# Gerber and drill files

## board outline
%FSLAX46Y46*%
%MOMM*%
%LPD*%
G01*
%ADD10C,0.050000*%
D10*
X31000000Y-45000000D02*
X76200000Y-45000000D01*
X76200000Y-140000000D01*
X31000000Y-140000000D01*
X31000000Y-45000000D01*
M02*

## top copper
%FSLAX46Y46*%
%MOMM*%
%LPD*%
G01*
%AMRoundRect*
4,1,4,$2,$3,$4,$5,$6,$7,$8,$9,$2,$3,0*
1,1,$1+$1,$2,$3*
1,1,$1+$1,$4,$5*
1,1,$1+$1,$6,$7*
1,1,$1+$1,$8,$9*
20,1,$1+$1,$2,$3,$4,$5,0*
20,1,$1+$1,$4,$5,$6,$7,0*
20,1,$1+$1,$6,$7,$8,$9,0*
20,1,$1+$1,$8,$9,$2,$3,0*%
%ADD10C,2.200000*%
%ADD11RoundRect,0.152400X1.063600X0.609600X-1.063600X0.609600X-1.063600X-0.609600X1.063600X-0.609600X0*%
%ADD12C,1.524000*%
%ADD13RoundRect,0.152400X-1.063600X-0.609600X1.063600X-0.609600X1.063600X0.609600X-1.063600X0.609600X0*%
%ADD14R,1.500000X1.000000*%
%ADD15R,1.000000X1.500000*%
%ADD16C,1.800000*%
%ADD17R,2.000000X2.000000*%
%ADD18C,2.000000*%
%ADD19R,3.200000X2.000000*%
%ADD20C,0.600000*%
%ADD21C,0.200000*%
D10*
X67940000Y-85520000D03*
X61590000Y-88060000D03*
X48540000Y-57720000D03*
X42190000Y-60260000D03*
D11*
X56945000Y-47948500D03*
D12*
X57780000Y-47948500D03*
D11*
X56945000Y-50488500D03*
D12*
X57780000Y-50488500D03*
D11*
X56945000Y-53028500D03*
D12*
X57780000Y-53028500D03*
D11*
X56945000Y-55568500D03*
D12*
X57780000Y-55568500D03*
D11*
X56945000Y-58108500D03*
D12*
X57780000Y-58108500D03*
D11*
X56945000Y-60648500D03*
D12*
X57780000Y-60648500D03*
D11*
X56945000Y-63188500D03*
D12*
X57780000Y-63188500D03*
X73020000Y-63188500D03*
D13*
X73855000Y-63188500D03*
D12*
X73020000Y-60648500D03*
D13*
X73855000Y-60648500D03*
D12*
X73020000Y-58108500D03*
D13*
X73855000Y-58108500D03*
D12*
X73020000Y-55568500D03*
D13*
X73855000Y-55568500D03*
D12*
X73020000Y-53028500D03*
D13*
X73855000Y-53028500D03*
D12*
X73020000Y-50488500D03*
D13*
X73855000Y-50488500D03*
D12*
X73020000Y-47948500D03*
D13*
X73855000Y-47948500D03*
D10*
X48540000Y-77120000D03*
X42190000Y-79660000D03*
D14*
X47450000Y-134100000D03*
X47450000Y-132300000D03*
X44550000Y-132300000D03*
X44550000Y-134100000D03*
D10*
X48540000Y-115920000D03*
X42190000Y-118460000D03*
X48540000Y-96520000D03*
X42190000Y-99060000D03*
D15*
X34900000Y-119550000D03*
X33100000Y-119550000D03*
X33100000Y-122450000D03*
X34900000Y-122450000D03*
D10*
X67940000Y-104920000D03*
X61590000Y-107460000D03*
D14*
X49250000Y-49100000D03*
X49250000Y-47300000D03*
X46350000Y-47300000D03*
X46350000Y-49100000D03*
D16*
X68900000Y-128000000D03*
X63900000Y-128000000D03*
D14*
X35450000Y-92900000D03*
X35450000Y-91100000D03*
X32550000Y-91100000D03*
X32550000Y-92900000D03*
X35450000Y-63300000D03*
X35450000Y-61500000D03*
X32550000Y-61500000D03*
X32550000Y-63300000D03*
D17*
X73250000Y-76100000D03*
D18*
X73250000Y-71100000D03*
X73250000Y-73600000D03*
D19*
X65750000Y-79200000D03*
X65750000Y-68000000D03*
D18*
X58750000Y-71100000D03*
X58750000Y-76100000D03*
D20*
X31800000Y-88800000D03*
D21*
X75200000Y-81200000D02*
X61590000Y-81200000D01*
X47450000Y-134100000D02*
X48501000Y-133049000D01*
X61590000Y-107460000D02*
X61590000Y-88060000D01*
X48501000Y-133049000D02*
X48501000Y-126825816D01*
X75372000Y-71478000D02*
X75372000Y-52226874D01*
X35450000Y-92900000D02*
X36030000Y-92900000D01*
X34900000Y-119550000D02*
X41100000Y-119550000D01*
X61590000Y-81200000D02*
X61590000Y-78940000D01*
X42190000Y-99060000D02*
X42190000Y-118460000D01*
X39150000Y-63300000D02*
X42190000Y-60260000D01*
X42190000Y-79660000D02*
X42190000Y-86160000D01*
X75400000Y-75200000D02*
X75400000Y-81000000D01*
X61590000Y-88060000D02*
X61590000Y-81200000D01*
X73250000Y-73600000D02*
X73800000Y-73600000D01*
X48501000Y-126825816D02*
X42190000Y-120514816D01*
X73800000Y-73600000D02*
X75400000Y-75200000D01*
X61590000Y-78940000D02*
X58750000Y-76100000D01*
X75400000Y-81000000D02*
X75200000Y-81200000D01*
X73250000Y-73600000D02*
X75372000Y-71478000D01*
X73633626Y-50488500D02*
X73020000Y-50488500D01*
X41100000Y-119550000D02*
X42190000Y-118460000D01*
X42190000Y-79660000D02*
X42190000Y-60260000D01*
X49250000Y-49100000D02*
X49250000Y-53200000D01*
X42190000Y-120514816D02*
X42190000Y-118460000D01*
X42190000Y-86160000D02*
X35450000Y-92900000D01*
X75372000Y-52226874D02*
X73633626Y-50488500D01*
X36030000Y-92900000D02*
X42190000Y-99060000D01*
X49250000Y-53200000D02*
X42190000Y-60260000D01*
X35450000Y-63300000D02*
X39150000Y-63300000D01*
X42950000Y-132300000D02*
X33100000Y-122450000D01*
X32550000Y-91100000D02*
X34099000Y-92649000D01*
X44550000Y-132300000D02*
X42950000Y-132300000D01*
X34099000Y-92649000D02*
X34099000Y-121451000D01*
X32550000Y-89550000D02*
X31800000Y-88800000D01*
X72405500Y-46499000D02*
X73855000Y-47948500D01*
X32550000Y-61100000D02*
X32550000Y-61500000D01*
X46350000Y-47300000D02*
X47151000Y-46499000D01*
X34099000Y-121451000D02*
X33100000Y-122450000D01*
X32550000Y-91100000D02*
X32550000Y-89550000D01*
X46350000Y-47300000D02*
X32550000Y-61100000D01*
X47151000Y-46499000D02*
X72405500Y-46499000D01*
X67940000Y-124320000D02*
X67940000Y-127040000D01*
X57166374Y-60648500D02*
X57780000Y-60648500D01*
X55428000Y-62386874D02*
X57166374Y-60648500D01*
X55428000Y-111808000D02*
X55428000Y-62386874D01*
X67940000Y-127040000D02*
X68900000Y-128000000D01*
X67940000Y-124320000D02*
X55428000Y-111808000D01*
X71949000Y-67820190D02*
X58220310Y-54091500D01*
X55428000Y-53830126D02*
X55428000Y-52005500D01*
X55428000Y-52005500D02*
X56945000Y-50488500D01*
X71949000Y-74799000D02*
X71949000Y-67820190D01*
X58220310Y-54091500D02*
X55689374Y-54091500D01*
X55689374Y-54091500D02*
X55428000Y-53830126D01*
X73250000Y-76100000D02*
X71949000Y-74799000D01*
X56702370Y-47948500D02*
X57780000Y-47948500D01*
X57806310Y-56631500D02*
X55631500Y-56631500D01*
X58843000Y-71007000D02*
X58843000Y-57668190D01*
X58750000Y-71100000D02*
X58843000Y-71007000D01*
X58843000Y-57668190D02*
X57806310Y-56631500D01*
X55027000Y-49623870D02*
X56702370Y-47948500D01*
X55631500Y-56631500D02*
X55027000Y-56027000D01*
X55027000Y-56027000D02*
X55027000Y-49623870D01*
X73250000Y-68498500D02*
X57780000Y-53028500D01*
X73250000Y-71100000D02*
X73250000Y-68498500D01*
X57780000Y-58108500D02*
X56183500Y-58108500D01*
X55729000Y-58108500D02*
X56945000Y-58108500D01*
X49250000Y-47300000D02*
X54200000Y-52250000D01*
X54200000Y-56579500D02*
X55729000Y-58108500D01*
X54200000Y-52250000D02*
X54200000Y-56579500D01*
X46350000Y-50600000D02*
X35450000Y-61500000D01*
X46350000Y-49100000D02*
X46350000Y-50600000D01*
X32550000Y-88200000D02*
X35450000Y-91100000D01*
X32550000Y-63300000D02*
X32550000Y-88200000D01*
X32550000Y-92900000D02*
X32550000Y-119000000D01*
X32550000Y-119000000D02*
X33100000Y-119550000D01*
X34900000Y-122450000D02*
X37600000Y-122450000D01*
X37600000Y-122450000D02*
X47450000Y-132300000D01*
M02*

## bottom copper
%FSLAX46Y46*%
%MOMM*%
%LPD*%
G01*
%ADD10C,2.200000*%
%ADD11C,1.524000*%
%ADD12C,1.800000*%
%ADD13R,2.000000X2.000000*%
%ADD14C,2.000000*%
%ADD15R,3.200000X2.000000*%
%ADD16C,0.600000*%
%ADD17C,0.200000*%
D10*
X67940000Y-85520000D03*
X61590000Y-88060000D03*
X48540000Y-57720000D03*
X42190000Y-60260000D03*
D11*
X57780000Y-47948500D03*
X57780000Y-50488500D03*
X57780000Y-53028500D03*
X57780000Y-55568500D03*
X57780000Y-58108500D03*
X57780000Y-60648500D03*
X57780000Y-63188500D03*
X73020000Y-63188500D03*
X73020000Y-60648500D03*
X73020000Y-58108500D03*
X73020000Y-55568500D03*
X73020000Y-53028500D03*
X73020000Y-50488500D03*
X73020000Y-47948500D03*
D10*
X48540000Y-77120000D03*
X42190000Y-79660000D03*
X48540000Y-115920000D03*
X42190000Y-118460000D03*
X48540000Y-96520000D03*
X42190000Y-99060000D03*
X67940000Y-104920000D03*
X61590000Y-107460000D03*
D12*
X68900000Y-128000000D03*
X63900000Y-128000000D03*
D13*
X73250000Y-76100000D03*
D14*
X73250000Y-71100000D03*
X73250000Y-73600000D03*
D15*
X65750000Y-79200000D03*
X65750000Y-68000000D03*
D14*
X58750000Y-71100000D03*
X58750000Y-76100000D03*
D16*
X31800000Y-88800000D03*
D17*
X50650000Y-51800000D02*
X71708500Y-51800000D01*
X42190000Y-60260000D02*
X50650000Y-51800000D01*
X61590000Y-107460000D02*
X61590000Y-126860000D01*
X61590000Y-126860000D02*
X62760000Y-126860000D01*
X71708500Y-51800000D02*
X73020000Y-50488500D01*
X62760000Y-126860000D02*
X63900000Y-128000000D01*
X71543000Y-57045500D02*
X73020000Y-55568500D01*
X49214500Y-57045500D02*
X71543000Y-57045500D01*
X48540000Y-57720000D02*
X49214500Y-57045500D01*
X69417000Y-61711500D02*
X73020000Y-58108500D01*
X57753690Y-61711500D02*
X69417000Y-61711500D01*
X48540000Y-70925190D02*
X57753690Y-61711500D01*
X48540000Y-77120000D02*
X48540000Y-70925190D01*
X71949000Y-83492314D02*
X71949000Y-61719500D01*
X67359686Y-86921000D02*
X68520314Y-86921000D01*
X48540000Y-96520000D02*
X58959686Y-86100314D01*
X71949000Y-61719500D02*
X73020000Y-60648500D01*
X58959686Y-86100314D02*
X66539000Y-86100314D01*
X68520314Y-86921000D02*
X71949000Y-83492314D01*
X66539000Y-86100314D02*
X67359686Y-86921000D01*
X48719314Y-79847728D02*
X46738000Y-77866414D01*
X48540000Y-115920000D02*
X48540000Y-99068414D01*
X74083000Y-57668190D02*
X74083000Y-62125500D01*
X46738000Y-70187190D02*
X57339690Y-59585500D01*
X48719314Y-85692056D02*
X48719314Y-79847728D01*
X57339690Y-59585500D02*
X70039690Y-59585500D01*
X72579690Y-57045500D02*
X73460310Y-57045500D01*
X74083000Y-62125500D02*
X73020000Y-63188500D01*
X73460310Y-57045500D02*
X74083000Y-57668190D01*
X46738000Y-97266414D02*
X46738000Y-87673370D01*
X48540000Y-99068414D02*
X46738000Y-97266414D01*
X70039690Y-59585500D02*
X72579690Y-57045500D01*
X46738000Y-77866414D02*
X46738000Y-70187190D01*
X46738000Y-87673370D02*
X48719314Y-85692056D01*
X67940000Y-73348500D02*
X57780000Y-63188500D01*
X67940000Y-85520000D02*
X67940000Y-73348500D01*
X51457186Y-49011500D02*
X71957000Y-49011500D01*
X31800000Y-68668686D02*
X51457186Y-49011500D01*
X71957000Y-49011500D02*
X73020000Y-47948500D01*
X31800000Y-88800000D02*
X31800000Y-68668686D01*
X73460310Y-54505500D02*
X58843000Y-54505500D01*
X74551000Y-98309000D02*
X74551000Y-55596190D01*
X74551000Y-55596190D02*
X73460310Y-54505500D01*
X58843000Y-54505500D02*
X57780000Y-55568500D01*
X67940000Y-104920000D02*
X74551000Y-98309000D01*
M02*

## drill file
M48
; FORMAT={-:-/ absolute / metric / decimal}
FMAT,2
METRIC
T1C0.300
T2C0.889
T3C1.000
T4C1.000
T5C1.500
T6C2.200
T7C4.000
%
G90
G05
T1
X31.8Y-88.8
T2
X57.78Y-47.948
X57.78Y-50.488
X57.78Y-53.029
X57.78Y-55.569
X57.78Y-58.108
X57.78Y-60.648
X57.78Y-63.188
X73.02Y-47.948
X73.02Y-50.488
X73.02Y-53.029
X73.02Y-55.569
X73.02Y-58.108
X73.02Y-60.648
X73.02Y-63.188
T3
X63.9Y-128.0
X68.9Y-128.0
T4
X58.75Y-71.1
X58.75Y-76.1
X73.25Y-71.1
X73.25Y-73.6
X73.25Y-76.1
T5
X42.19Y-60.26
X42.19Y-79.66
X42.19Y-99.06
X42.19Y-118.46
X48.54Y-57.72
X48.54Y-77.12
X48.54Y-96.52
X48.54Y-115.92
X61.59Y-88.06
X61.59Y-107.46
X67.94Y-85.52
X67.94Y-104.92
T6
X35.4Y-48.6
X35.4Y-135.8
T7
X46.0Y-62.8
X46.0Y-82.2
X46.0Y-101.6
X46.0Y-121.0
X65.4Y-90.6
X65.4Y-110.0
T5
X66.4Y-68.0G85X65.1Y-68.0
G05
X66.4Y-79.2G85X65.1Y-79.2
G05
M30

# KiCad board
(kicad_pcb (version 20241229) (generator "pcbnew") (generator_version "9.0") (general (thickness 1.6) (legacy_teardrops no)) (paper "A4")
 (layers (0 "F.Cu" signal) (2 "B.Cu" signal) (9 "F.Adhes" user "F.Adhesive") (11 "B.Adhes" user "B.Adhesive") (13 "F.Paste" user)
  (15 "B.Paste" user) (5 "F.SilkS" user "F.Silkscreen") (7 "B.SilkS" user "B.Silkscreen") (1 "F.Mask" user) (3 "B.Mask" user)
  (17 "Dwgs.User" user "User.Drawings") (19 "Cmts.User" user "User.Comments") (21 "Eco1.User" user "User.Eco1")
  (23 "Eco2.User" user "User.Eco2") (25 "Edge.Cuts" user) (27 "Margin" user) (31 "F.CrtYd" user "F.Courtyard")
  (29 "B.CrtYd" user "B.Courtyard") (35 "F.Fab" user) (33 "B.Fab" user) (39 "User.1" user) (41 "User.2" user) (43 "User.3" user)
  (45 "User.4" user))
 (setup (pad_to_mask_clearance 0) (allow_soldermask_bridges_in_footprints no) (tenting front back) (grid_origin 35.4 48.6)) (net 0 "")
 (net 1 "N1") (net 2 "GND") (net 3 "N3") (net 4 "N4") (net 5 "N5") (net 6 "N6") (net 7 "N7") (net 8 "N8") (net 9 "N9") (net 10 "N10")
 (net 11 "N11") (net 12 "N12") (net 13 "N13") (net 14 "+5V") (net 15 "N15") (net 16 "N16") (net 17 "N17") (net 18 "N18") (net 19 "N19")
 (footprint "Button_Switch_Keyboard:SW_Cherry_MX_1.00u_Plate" (layer "F.Cu") (at 67.94 85.52)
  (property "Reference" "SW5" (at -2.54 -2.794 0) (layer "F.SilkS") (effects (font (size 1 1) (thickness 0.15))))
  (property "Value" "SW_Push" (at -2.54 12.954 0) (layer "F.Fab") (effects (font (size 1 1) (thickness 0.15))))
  (pad "" np_thru_hole circle (at -2.54 5.08) (size 4 4) (drill 4) (layers "*.Cu" "*.Mask"))
  (pad "1" thru_hole circle (at 0 0) (size 2.2 2.2) (drill 1.5) (layers "*.Cu" "*.Mask") (remove_unused_layers no) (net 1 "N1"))
  (pad "2" thru_hole circle (at -6.35 2.54) (size 2.2 2.2) (drill 1.5) (layers "*.Cu" "*.Mask") (remove_unused_layers no) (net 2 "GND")))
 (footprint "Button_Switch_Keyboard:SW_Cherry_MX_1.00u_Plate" (layer "F.Cu") (at 48.54 57.72)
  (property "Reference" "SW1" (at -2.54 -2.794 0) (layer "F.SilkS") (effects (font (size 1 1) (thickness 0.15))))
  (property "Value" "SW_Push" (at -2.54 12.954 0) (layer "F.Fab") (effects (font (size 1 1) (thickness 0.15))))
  (pad "" np_thru_hole circle (at -2.54 5.08) (size 4 4) (drill 4) (layers "*.Cu" "*.Mask"))
  (pad "1" thru_hole circle (at 0 0) (size 2.2 2.2) (drill 1.5) (layers "*.Cu" "*.Mask") (remove_unused_layers no) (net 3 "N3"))
  (pad "2" thru_hole circle (at -6.35 2.54) (size 2.2 2.2) (drill 1.5) (layers "*.Cu" "*.Mask") (remove_unused_layers no) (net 2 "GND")))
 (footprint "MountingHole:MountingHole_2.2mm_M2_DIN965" (layer "F.Cu") (at 35.4 135.8)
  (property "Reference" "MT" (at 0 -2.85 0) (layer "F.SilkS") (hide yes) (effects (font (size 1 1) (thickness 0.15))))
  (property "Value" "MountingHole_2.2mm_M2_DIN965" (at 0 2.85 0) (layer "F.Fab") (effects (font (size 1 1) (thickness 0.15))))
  (pad "" np_thru_hole circle (at 0 0) (size 2.2 2.2) (drill 2.2) (layers "*.Cu" "*.Mask")))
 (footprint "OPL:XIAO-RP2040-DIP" (layer "F.Cu") (at 65.4 55.5685)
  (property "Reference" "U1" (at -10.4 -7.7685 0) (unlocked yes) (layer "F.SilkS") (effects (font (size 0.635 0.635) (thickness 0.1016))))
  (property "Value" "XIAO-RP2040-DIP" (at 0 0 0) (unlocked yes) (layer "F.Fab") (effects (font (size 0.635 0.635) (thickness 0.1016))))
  (pad "1" smd roundrect (at -8.455 -7.62 180) (size 2.432 1.524) (layers "F.Cu" "F.Mask") (roundrect_rratio 0.1) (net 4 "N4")
   (thermal_bridge_angle 45))
  (pad "1" thru_hole circle (at -7.62 -7.62 180) (size 1.524 1.524) (drill 0.889) (layers "*.Cu" "*.Mask") (remove_unused_layers no)
   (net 4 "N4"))
  (pad "2" smd roundrect (at -8.455 -5.08 180) (size 2.432 1.524) (layers "F.Cu" "F.Mask") (roundrect_rratio 0.1) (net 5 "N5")
   (thermal_bridge_angle 45))
  (pad "2" thru_hole circle (at -7.62 -5.08 180) (size 1.524 1.524) (drill 0.889) (layers "*.Cu" "*.Mask") (remove_unused_layers no)
   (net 5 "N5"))
  (pad "3" smd roundrect (at -8.455 -2.54 180) (size 2.432 1.524) (layers "F.Cu" "F.Mask") (roundrect_rratio 0.1) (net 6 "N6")
   (thermal_bridge_angle 45))
  (pad "3" thru_hole circle (at -7.62 -2.54 180) (size 1.524 1.524) (drill 0.889) (layers "*.Cu" "*.Mask") (remove_unused_layers no)
   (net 6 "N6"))
  (pad "4" smd roundrect (at -8.455 0 180) (size 2.432 1.524) (layers "F.Cu" "F.Mask") (roundrect_rratio 0.1) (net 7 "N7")
   (thermal_bridge_angle 45))
  (pad "4" thru_hole circle (at -7.62 0 180) (size 1.524 1.524) (drill 0.889) (layers "*.Cu" "*.Mask") (remove_unused_layers no)
   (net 7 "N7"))
  (pad "5" smd roundrect (at -8.455 2.54 180) (size 2.432 1.524) (layers "F.Cu" "F.Mask") (roundrect_rratio 0.1) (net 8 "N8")
   (thermal_bridge_angle 45))
  (pad "5" thru_hole circle (at -7.62 2.54 180) (size 1.524 1.524) (drill 0.889) (layers "*.Cu" "*.Mask") (remove_unused_layers no)
   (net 8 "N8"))
  (pad "6" smd roundrect (at -8.455 5.08 180) (size 2.432 1.524) (layers "F.Cu" "F.Mask") (roundrect_rratio 0.1) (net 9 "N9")
   (thermal_bridge_angle 45))
  (pad "6" thru_hole circle (at -7.62 5.08 180) (size 1.524 1.524) (drill 0.889) (layers "*.Cu" "*.Mask") (remove_unused_layers no)
   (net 9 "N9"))
  (pad "7" smd roundrect (at -8.455 7.62 180) (size 2.432 1.524) (layers "F.Cu" "F.Mask") (roundrect_rratio 0.1) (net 1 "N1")
   (thermal_bridge_angle 45))
  (pad "7" thru_hole circle (at -7.62 7.62 180) (size 1.524 1.524) (drill 0.889) (layers "*.Cu" "*.Mask") (remove_unused_layers no)
   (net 1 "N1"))
  (pad "8" thru_hole circle (at 7.62 7.62) (size 1.524 1.524) (drill 0.889) (layers "*.Cu" "*.Mask") (remove_unused_layers no)
   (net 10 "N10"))
  (pad "8" smd roundrect (at 8.455 7.62) (size 2.432 1.524) (layers "F.Cu" "F.Mask") (roundrect_rratio 0.1) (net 10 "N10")
   (thermal_bridge_angle 45))
  (pad "9" thru_hole circle (at 7.62 5.08) (size 1.524 1.524) (drill 0.889) (layers "*.Cu" "*.Mask") (remove_unused_layers no)
   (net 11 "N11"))
  (pad "9" smd roundrect (at 8.455 5.08) (size 2.432 1.524) (layers "F.Cu" "F.Mask") (roundrect_rratio 0.1) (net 11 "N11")
   (thermal_bridge_angle 45))
  (pad "10" thru_hole circle (at 7.62 2.54) (size 1.524 1.524) (drill 0.889) (layers "*.Cu" "*.Mask") (remove_unused_layers no)
   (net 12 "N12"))
  (pad "10" smd roundrect (at 8.455 2.54) (size 2.432 1.524) (layers "F.Cu" "F.Mask") (roundrect_rratio 0.1) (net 12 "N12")
   (thermal_bridge_angle 45))
  (pad "11" thru_hole circle (at 7.62 0) (size 1.524 1.524) (drill 0.889) (layers "*.Cu" "*.Mask") (remove_unused_layers no) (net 3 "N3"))
  (pad "11" smd roundrect (at 8.455 0) (size 2.432 1.524) (layers "F.Cu" "F.Mask") (roundrect_rratio 0.1) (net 3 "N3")
   (thermal_bridge_angle 45))
  (pad "12" thru_hole circle (at 7.62 -2.54) (size 1.524 1.524) (drill 0.889) (layers "*.Cu" "*.Mask") (remove_unused_layers no)
   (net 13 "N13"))
  (pad "12" smd roundrect (at 8.455 -2.54) (size 2.432 1.524) (layers "F.Cu" "F.Mask") (roundrect_rratio 0.1) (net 13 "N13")
   (thermal_bridge_angle 45))
  (pad "13" thru_hole circle (at 7.62 -5.08) (size 1.524 1.524) (drill 0.889) (layers "*.Cu" "*.Mask") (remove_unused_layers no)
   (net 2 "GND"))
  (pad "13" smd roundrect (at 8.455 -5.08) (size 2.432 1.524) (layers "F.Cu" "F.Mask") (roundrect_rratio 0.1) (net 2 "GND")
   (thermal_bridge_angle 45))
  (pad "14" thru_hole circle (at 7.62 -7.62) (size 1.524 1.524) (drill 0.889) (layers "*.Cu" "*.Mask") (remove_unused_layers no)
   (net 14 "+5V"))
  (pad "14" smd roundrect (at 8.455 -7.62) (size 2.432 1.524) (layers "F.Cu" "F.Mask") (roundrect_rratio 0.1) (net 14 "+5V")
   (thermal_bridge_angle 45)))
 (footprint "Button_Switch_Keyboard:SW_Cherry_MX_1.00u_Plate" (layer "F.Cu") (at 48.54 77.12)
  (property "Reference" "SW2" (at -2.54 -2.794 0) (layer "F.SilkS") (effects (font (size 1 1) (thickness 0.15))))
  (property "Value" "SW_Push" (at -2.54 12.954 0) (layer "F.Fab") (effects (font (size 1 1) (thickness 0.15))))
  (pad "" np_thru_hole circle (at -2.54 5.08) (size 4 4) (drill 4) (layers "*.Cu" "*.Mask"))
  (pad "1" thru_hole circle (at 0 0) (size 2.2 2.2) (drill 1.5) (layers "*.Cu" "*.Mask") (remove_unused_layers no) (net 12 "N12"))
  (pad "2" thru_hole circle (at -6.35 2.54) (size 2.2 2.2) (drill 1.5) (layers "*.Cu" "*.Mask") (remove_unused_layers no) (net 2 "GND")))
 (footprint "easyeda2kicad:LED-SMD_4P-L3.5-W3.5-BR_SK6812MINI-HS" (layer "F.Cu") (at 46 133.2)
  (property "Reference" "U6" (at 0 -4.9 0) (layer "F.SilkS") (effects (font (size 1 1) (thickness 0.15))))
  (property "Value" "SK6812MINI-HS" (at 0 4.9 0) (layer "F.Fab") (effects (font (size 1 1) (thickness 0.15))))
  (pad "1" smd rect (at 1.45 0.9 180) (size 1.5 1) (layers "F.Cu" "F.Mask" "F.Paste") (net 2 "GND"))
  (pad "2" smd rect (at 1.45 -0.9 180) (size 1.5 1) (layers "F.Cu" "F.Mask" "F.Paste") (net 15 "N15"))
  (pad "3" smd rect (at -1.45 -0.9 180) (size 1.5 1) (layers "F.Cu" "F.Mask" "F.Paste") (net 14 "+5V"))
  (pad "4" smd rect (at -1.45 0.9 180) (size 1.5 1) (layers "F.Cu" "F.Mask" "F.Paste") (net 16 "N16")))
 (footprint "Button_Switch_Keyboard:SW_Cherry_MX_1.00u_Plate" (layer "F.Cu") (at 48.54 115.92)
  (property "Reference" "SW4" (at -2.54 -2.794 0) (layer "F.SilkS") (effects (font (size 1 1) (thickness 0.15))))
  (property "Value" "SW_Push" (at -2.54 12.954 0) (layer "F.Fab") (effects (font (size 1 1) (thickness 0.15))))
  (pad "" np_thru_hole circle (at -2.54 5.08) (size 4 4) (drill 4) (layers "*.Cu" "*.Mask"))
  (pad "1" thru_hole circle (at 0 0) (size 2.2 2.2) (drill 1.5) (layers "*.Cu" "*.Mask") (remove_unused_layers no) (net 10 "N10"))
  (pad "2" thru_hole circle (at -6.35 2.54) (size 2.2 2.2) (drill 1.5) (layers "*.Cu" "*.Mask") (remove_unused_layers no) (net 2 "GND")))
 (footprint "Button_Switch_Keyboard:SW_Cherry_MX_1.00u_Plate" (layer "F.Cu") (at 48.54 96.52)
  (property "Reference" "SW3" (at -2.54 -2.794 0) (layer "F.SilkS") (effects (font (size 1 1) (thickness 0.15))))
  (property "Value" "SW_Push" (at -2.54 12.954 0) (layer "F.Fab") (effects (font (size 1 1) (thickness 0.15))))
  (pad "" np_thru_hole circle (at -2.54 5.08) (size 4 4) (drill 4) (layers "*.Cu" "*.Mask"))
  (pad "1" thru_hole circle (at 0 0) (size 2.2 2.2) (drill 1.5) (layers "*.Cu" "*.Mask") (remove_unused_layers no) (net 11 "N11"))
  (pad "2" thru_hole circle (at -6.35 2.54) (size 2.2 2.2) (drill 1.5) (layers "*.Cu" "*.Mask") (remove_unused_layers no) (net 2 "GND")))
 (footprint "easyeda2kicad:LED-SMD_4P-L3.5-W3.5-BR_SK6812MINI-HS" (layer "F.Cu") (at 34 121 90)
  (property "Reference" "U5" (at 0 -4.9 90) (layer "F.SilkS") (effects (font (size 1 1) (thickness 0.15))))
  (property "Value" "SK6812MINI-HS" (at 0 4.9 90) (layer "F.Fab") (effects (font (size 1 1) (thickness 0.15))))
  (pad "1" smd rect (at 1.45 0.9 270) (size 1.5 1) (layers "F.Cu" "F.Mask" "F.Paste") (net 2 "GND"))
  (pad "2" smd rect (at 1.45 -0.9 270) (size 1.5 1) (layers "F.Cu" "F.Mask" "F.Paste") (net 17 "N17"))
  (pad "3" smd rect (at -1.45 -0.9 270) (size 1.5 1) (layers "F.Cu" "F.Mask" "F.Paste") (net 14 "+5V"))
  (pad "4" smd rect (at -1.45 0.9 270) (size 1.5 1) (layers "F.Cu" "F.Mask" "F.Paste") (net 15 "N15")))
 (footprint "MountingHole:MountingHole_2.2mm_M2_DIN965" (layer "F.Cu") (at 35.4 48.6)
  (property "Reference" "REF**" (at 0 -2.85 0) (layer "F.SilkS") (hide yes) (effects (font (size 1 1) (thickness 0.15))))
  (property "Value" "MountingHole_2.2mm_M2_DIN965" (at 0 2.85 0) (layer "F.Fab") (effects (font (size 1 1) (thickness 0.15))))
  (pad "" np_thru_hole circle (at 0 0) (size 2.2 2.2) (drill 2.2) (layers "*.Cu" "*.Mask")))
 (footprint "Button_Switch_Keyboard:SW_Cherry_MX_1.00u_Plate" (layer "F.Cu") (at 67.94 104.92)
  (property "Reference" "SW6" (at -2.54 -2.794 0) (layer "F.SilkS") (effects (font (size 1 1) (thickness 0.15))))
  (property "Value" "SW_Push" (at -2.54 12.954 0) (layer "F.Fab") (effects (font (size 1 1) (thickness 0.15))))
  (pad "" np_thru_hole circle (at -2.54 5.08) (size 4 4) (drill 4) (layers "*.Cu" "*.Mask"))
  (pad "1" thru_hole circle (at 0 0) (size 2.2 2.2) (drill 1.5) (layers "*.Cu" "*.Mask") (remove_unused_layers no) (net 7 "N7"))
  (pad "2" thru_hole circle (at -6.35 2.54) (size 2.2 2.2) (drill 1.5) (layers "*.Cu" "*.Mask") (remove_unused_layers no) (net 2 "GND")))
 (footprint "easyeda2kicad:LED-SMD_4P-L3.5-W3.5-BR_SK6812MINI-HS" (layer "F.Cu") (at 47.8 48.2)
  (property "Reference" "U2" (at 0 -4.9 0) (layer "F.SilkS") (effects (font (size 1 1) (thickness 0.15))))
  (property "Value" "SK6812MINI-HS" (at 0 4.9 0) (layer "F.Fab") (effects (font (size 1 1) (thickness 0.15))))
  (pad "1" smd rect (at 1.45 0.9 180) (size 1.5 1) (layers "F.Cu" "F.Mask" "F.Paste") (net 2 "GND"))
  (pad "2" smd rect (at 1.45 -0.9 180) (size 1.5 1) (layers "F.Cu" "F.Mask" "F.Paste") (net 8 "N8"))
  (pad "3" smd rect (at -1.45 -0.9 180) (size 1.5 1) (layers "F.Cu" "F.Mask" "F.Paste") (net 14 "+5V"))
  (pad "4" smd rect (at -1.45 0.9 180) (size 1.5 1) (layers "F.Cu" "F.Mask" "F.Paste") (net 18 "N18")))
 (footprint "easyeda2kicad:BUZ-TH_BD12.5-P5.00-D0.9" (layer "F.Cu") (at 66.4 128 180)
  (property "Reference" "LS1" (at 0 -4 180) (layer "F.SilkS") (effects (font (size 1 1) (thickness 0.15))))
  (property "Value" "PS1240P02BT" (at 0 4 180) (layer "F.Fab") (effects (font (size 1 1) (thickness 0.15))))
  (pad "1" thru_hole circle (at -2.5 0 180) (size 1.8 1.8) (drill 0.999998) (layers "*.Cu" "*.Mask") (remove_unused_layers no) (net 9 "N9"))
  (pad "2" thru_hole circle (at 2.5 0 180) (size 1.8 1.8) (drill 0.999998) (layers "*.Cu" "*.Mask") (remove_unused_layers no) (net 2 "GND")))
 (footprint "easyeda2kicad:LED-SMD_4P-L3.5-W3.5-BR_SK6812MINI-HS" (layer "F.Cu") (at 34 92)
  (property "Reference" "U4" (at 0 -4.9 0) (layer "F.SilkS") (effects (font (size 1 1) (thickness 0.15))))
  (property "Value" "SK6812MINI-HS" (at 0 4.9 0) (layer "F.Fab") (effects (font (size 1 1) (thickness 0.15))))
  (pad "1" smd rect (at 1.45 0.9 180) (size 1.5 1) (layers "F.Cu" "F.Mask" "F.Paste") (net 2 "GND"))
  (pad "2" smd rect (at 1.45 -0.9 180) (size 1.5 1) (layers "F.Cu" "F.Mask" "F.Paste") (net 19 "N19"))
  (pad "3" smd rect (at -1.45 -0.9 180) (size 1.5 1) (layers "F.Cu" "F.Mask" "F.Paste") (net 14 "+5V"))
  (pad "4" smd rect (at -1.45 0.9 180) (size 1.5 1) (layers "F.Cu" "F.Mask" "F.Paste") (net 17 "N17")))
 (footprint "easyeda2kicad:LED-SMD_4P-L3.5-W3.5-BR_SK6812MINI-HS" (layer "F.Cu") (at 34 62.4)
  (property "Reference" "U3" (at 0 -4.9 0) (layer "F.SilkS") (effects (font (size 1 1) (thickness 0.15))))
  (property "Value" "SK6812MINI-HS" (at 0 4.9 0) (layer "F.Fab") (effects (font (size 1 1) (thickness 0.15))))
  (pad "1" smd rect (at 1.45 0.9 180) (size 1.5 1) (layers "F.Cu" "F.Mask" "F.Paste") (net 2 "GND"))
  (pad "2" smd rect (at 1.45 -0.9 180) (size 1.5 1) (layers "F.Cu" "F.Mask" "F.Paste") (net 18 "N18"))
  (pad "3" smd rect (at -1.45 -0.9 180) (size 1.5 1) (layers "F.Cu" "F.Mask" "F.Paste") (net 14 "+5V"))
  (pad "4" smd rect (at -1.45 0.9 180) (size 1.5 1) (layers "F.Cu" "F.Mask" "F.Paste") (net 19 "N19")))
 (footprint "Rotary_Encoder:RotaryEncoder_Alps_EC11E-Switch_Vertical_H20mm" (layer "F.Cu") (at 73.25 76.1 180)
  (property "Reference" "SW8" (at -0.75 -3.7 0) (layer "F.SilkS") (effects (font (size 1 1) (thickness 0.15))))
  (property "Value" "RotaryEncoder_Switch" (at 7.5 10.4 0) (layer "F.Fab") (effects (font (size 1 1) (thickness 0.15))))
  (pad "A" thru_hole rect (at 0 0 180) (size 2 2) (drill 1) (layers "*.Cu" "*.Mask") (remove_unused_layers no) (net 5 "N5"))
  (pad "B" thru_hole circle (at 0 5 180) (size 2 2) (drill 1) (layers "*.Cu" "*.Mask") (remove_unused_layers no) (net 6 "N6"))
  (pad "C" thru_hole circle (at 0 2.5 180) (size 2 2) (drill 1) (layers "*.Cu" "*.Mask") (remove_unused_layers no) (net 2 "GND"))
  (pad "MP" thru_hole rect (at 7.5 -3.1 180) (size 3.2 2) (drill oval 2.8 1.5) (layers "*.Cu" "*.Mask") (remove_unused_layers no))
  (pad "MP" thru_hole rect (at 7.5 8.1 180) (size 3.2 2) (drill oval 2.8 1.5) (layers "*.Cu" "*.Mask") (remove_unused_layers no))
  (pad "S1" thru_hole circle (at 14.5 5 180) (size 2 2) (drill 1) (layers "*.Cu" "*.Mask") (remove_unused_layers no) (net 4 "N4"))
  (pad "S2" thru_hole circle (at 14.5 0 180) (size 2 2) (drill 1) (layers "*.Cu" "*.Mask") (remove_unused_layers no) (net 2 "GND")))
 (gr_rect (start 31 45) (end 76.2 140) (stroke (width 0.05) (type default)) (fill no) (layer "Edge.Cuts"))
 (segment (start 75.2 81.2) (end 61.59 81.2) (width 0.2) (layer "F.Cu") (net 2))
 (segment (start 47.45 134.1) (end 48.501 133.049) (width 0.2) (layer "F.Cu") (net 2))
 (segment (start 61.59 107.46) (end 61.59 88.06) (width 0.2) (layer "F.Cu") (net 2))
 (segment (start 48.501 133.049) (end 48.501 126.825816) (width 0.2) (layer "F.Cu") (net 2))
 (segment (start 75.372 71.478) (end 75.372 52.226874) (width 0.2) (layer "F.Cu") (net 2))
 (segment (start 35.45 92.9) (end 36.03 92.9) (width 0.2) (layer "F.Cu") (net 2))
 (segment (start 34.9 119.55) (end 41.1 119.55) (width 0.2) (layer "F.Cu") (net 2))
 (segment (start 61.59 81.2) (end 61.59 78.94) (width 0.2) (layer "F.Cu") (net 2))
 (segment (start 42.19 99.06) (end 42.19 118.46) (width 0.2) (layer "F.Cu") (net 2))
 (segment (start 39.15 63.3) (end 42.19 60.26) (width 0.2) (layer "F.Cu") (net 2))
 (segment (start 42.19 79.66) (end 42.19 86.16) (width 0.2) (layer "F.Cu") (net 2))
 (segment (start 75.4 75.2) (end 75.4 81) (width 0.2) (layer "F.Cu") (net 2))
 (segment (start 61.59 88.06) (end 61.59 81.2) (width 0.2) (layer "F.Cu") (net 2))
 (segment (start 73.25 73.6) (end 73.8 73.6) (width 0.2) (layer "F.Cu") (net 2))
 (segment (start 48.501 126.825816) (end 42.19 120.514816) (width 0.2) (layer "F.Cu") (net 2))
 (segment (start 73.8 73.6) (end 75.4 75.2) (width 0.2) (layer "F.Cu") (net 2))
 (segment (start 61.59 78.94) (end 58.75 76.1) (width 0.2) (layer "F.Cu") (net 2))
 (segment (start 75.4 81) (end 75.2 81.2) (width 0.2) (layer "F.Cu") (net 2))
 (segment (start 73.25 73.6) (end 75.372 71.478) (width 0.2) (layer "F.Cu") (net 2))
 (segment (start 73.633626 50.4885) (end 73.02 50.4885) (width 0.2) (layer "F.Cu") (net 2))
 (segment (start 41.1 119.55) (end 42.19 118.46) (width 0.2) (layer "F.Cu") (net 2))
 (segment (start 42.19 79.66) (end 42.19 60.26) (width 0.2) (layer "F.Cu") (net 2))
 (segment (start 49.25 49.1) (end 49.25 53.2) (width 0.2) (layer "F.Cu") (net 2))
 (segment (start 42.19 120.514816) (end 42.19 118.46) (width 0.2) (layer "F.Cu") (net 2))
 (segment (start 42.19 86.16) (end 35.45 92.9) (width 0.2) (layer "F.Cu") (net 2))
 (segment (start 75.372 52.226874) (end 73.633626 50.4885) (width 0.2) (layer "F.Cu") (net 2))
 (segment (start 36.03 92.9) (end 42.19 99.06) (width 0.2) (layer "F.Cu") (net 2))
 (segment (start 49.25 53.2) (end 42.19 60.26) (width 0.2) (layer "F.Cu") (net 2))
 (segment (start 35.45 63.3) (end 39.15 63.3) (width 0.2) (layer "F.Cu") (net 2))
 (segment (start 50.65 51.8) (end 71.7085 51.8) (width 0.2) (layer "B.Cu") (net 2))
 (segment (start 42.19 60.26) (end 50.65 51.8) (width 0.2) (layer "B.Cu") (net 2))
 (segment (start 61.59 107.46) (end 61.59 126.86) (width 0.2) (layer "B.Cu") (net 2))
 (segment (start 61.59 126.86) (end 62.76 126.86) (width 0.2) (layer "B.Cu") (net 2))
 (segment (start 71.7085 51.8) (end 73.02 50.4885) (width 0.2) (layer "B.Cu") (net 2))
 (segment (start 62.76 126.86) (end 63.9 128) (width 0.2) (layer "B.Cu") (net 2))
 (segment (start 71.543 57.0455) (end 73.02 55.5685) (width 0.2) (layer "B.Cu") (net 3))
 (segment (start 49.2145 57.0455) (end 71.543 57.0455) (width 0.2) (layer "B.Cu") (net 3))
 (segment (start 48.54 57.72) (end 49.2145 57.0455) (width 0.2) (layer "B.Cu") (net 3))
 (segment (start 69.417 61.7115) (end 73.02 58.1085) (width 0.2) (layer "B.Cu") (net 12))
 (segment (start 57.75369 61.7115) (end 69.417 61.7115) (width 0.2) (layer "B.Cu") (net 12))
 (segment (start 48.54 70.92519) (end 57.75369 61.7115) (width 0.2) (layer "B.Cu") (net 12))
 (segment (start 48.54 77.12) (end 48.54 70.92519) (width 0.2) (layer "B.Cu") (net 12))
 (segment (start 71.949 83.492314) (end 71.949 61.7195) (width 0.2) (layer "B.Cu") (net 11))
 (segment (start 67.359686 86.921) (end 68.520314 86.921) (width 0.2) (layer "B.Cu") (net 11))
 (segment (start 48.54 96.52) (end 58.959686 86.100314) (width 0.2) (layer "B.Cu") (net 11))
 (segment (start 71.949 61.7195) (end 73.02 60.6485) (width 0.2) (layer "B.Cu") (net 11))
 (segment (start 58.959686 86.100314) (end 66.539 86.100314) (width 0.2) (layer "B.Cu") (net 11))
 (segment (start 68.520314 86.921) (end 71.949 83.492314) (width 0.2) (layer "B.Cu") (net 11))
 (segment (start 66.539 86.100314) (end 67.359686 86.921) (width 0.2) (layer "B.Cu") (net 11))
 (segment (start 48.719314 79.847728) (end 46.738 77.866414) (width 0.2) (layer "B.Cu") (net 10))
 (segment (start 48.54 115.92) (end 48.54 99.068414) (width 0.2) (layer "B.Cu") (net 10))
 (segment (start 74.083 57.66819) (end 74.083 62.1255) (width 0.2) (layer "B.Cu") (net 10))
 (segment (start 46.738 70.18719) (end 57.33969 59.5855) (width 0.2) (layer "B.Cu") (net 10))
 (segment (start 48.719314 85.692056) (end 48.719314 79.847728) (width 0.2) (layer "B.Cu") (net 10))
 (segment (start 57.33969 59.5855) (end 70.03969 59.5855) (width 0.2) (layer "B.Cu") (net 10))
 (segment (start 72.57969 57.0455) (end 73.46031 57.0455) (width 0.2) (layer "B.Cu") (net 10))
 (segment (start 74.083 62.1255) (end 73.02 63.1885) (width 0.2) (layer "B.Cu") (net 10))
 (segment (start 73.46031 57.0455) (end 74.083 57.66819) (width 0.2) (layer "B.Cu") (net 10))
 (segment (start 46.738 97.266414) (end 46.738 87.67337) (width 0.2) (layer "B.Cu") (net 10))
 (segment (start 48.54 99.068414) (end 46.738 97.266414) (width 0.2) (layer "B.Cu") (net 10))
 (segment (start 70.03969 59.5855) (end 72.57969 57.0455) (width 0.2) (layer "B.Cu") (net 10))
 (segment (start 46.738 77.866414) (end 46.738 70.18719) (width 0.2) (layer "B.Cu") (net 10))
 (segment (start 46.738 87.67337) (end 48.719314 85.692056) (width 0.2) (layer "B.Cu") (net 10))
 (segment (start 67.94 73.3485) (end 57.78 63.1885) (width 0.2) (layer "B.Cu") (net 1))
 (segment (start 67.94 85.52) (end 67.94 73.3485) (width 0.2) (layer "B.Cu") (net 1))
 (segment (start 42.95 132.3) (end 33.1 122.45) (width 0.2) (layer "F.Cu") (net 14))
 (segment (start 32.55 91.1) (end 34.099 92.649) (width 0.2) (layer "F.Cu") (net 14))
 (segment (start 44.55 132.3) (end 42.95 132.3) (width 0.2) (layer "F.Cu") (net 14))
 (segment (start 34.099 92.649) (end 34.099 121.451) (width 0.2) (layer "F.Cu") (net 14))
 (segment (start 32.55 89.55) (end 31.8 88.8) (width 0.2) (layer "F.Cu") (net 14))
 (segment (start 72.4055 46.499) (end 73.855 47.9485) (width 0.2) (layer "F.Cu") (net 14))
 (segment (start 32.55 61.1) (end 32.55 61.5) (width 0.2) (layer "F.Cu") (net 14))
 (segment (start 46.35 47.3) (end 47.151 46.499) (width 0.2) (layer "F.Cu") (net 14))
 (segment (start 34.099 121.451) (end 33.1 122.45) (width 0.2) (layer "F.Cu") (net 14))
 (segment (start 32.55 91.1) (end 32.55 89.55) (width 0.2) (layer "F.Cu") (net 14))
 (segment (start 46.35 47.3) (end 32.55 61.1) (width 0.2) (layer "F.Cu") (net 14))
 (segment (start 47.151 46.499) (end 72.4055 46.499) (width 0.2) (layer "F.Cu") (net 14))
 (via (at 31.8 88.8) (size 0.6) (drill 0.3) (layers "F.Cu" "B.Cu") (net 14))
 (segment (start 51.457186 49.0115) (end 71.957 49.0115) (width 0.2) (layer "B.Cu") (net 14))
 (segment (start 31.8 68.668686) (end 51.457186 49.0115) (width 0.2) (layer "B.Cu") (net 14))
 (segment (start 71.957 49.0115) (end 73.02 47.9485) (width 0.2) (layer "B.Cu") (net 14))
 (segment (start 31.8 88.8) (end 31.8 68.668686) (width 0.2) (layer "B.Cu") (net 14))
 (segment (start 73.46031 54.5055) (end 58.843 54.5055) (width 0.2) (layer "B.Cu") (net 7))
 (segment (start 74.551 98.309) (end 74.551 55.59619) (width 0.2) (layer "B.Cu") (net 7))
 (segment (start 74.551 55.59619) (end 73.46031 54.5055) (width 0.2) (layer "B.Cu") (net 7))
 (segment (start 58.843 54.5055) (end 57.78 55.5685) (width 0.2) (layer "B.Cu") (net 7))
 (segment (start 67.94 104.92) (end 74.551 98.309) (width 0.2) (layer "B.Cu") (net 7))
 (segment (start 67.94 124.32) (end 67.94 127.04) (width 0.2) (layer "F.Cu") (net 9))
 (segment (start 57.166374 60.6485) (end 57.78 60.6485) (width 0.2) (layer "F.Cu") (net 9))
 (segment (start 55.428 62.386874) (end 57.166374 60.6485) (width 0.2) (layer "F.Cu") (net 9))
 (segment (start 55.428 111.808) (end 55.428 62.386874) (width 0.2) (layer "F.Cu") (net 9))
 (segment (start 67.94 127.04) (end 68.9 128) (width 0.2) (layer "F.Cu") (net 9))
 (segment (start 67.94 124.32) (end 55.428 111.808) (width 0.2) (layer "F.Cu") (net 9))
 (segment (start 71.949 67.82019) (end 58.22031 54.0915) (width 0.2) (layer "F.Cu") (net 5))
 (segment (start 55.428 53.830126) (end 55.428 52.0055) (width 0.2) (layer "F.Cu") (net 5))
 (segment (start 55.428 52.0055) (end 56.945 50.4885) (width 0.2) (layer "F.Cu") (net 5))
 (segment (start 71.949 74.799) (end 71.949 67.82019) (width 0.2) (layer "F.Cu") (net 5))
 (segment (start 58.22031 54.0915) (end 55.689374 54.0915) (width 0.2) (layer "F.Cu") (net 5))
 (segment (start 55.689374 54.0915) (end 55.428 53.830126) (width 0.2) (layer "F.Cu") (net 5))
 (segment (start 73.25 76.1) (end 71.949 74.799) (width 0.2) (layer "F.Cu") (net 5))
 (segment (start 56.70237 47.9485) (end 57.78 47.9485) (width 0.2) (layer "F.Cu") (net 4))
 (segment (start 57.80631 56.6315) (end 55.6315 56.6315) (width 0.2) (layer "F.Cu") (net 4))
 (segment (start 58.843 71.007) (end 58.843 57.66819) (width 0.2) (layer "F.Cu") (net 4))
 (segment (start 58.75 71.1) (end 58.843 71.007) (width 0.2) (layer "F.Cu") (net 4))
 (segment (start 58.843 57.66819) (end 57.80631 56.6315) (width 0.2) (layer "F.Cu") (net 4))
 (segment (start 55.027 49.62387) (end 56.70237 47.9485) (width 0.2) (layer "F.Cu") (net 4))
 (segment (start 55.6315 56.6315) (end 55.027 56.027) (width 0.2) (layer "F.Cu") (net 4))
 (segment (start 55.027 56.027) (end 55.027 49.62387) (width 0.2) (layer "F.Cu") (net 4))
 (segment (start 73.25 68.4985) (end 57.78 53.0285) (width 0.2) (layer "F.Cu") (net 6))
 (segment (start 73.25 71.1) (end 73.25 68.4985) (width 0.2) (layer "F.Cu") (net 6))
 (segment (start 57.78 58.1085) (end 56.1835 58.1085) (width 0.2) (layer "F.Cu") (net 8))
 (segment (start 55.729 58.1085) (end 56.945 58.1085) (width 0.2) (layer "F.Cu") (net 8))
 (segment (start 49.25 47.3) (end 54.2 52.25) (width 0.2) (layer "F.Cu") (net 8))
 (segment (start 54.2 56.5795) (end 55.729 58.1085) (width 0.2) (layer "F.Cu") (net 8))
 (segment (start 54.2 52.25) (end 54.2 56.5795) (width 0.2) (layer "F.Cu") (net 8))
 (segment (start 46.35 50.6) (end 35.45 61.5) (width 0.2) (layer "F.Cu") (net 18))
 (segment (start 46.35 49.1) (end 46.35 50.6) (width 0.2) (layer "F.Cu") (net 18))
 (segment (start 32.55 88.2) (end 35.45 91.1) (width 0.2) (layer "F.Cu") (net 19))
 (segment (start 32.55 63.3) (end 32.55 88.2) (width 0.2) (layer "F.Cu") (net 19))
 (segment (start 32.55 92.9) (end 32.55 119) (width 0.2) (layer "F.Cu") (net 17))
 (segment (start 32.55 119) (end 33.1 119.55) (width 0.2) (layer "F.Cu") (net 17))
 (segment (start 34.9 122.45) (end 37.6 122.45) (width 0.2) (layer "F.Cu") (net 15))
 (segment (start 37.6 122.45) (end 47.45 132.3) (width 0.2) (layer "F.Cu") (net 15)))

